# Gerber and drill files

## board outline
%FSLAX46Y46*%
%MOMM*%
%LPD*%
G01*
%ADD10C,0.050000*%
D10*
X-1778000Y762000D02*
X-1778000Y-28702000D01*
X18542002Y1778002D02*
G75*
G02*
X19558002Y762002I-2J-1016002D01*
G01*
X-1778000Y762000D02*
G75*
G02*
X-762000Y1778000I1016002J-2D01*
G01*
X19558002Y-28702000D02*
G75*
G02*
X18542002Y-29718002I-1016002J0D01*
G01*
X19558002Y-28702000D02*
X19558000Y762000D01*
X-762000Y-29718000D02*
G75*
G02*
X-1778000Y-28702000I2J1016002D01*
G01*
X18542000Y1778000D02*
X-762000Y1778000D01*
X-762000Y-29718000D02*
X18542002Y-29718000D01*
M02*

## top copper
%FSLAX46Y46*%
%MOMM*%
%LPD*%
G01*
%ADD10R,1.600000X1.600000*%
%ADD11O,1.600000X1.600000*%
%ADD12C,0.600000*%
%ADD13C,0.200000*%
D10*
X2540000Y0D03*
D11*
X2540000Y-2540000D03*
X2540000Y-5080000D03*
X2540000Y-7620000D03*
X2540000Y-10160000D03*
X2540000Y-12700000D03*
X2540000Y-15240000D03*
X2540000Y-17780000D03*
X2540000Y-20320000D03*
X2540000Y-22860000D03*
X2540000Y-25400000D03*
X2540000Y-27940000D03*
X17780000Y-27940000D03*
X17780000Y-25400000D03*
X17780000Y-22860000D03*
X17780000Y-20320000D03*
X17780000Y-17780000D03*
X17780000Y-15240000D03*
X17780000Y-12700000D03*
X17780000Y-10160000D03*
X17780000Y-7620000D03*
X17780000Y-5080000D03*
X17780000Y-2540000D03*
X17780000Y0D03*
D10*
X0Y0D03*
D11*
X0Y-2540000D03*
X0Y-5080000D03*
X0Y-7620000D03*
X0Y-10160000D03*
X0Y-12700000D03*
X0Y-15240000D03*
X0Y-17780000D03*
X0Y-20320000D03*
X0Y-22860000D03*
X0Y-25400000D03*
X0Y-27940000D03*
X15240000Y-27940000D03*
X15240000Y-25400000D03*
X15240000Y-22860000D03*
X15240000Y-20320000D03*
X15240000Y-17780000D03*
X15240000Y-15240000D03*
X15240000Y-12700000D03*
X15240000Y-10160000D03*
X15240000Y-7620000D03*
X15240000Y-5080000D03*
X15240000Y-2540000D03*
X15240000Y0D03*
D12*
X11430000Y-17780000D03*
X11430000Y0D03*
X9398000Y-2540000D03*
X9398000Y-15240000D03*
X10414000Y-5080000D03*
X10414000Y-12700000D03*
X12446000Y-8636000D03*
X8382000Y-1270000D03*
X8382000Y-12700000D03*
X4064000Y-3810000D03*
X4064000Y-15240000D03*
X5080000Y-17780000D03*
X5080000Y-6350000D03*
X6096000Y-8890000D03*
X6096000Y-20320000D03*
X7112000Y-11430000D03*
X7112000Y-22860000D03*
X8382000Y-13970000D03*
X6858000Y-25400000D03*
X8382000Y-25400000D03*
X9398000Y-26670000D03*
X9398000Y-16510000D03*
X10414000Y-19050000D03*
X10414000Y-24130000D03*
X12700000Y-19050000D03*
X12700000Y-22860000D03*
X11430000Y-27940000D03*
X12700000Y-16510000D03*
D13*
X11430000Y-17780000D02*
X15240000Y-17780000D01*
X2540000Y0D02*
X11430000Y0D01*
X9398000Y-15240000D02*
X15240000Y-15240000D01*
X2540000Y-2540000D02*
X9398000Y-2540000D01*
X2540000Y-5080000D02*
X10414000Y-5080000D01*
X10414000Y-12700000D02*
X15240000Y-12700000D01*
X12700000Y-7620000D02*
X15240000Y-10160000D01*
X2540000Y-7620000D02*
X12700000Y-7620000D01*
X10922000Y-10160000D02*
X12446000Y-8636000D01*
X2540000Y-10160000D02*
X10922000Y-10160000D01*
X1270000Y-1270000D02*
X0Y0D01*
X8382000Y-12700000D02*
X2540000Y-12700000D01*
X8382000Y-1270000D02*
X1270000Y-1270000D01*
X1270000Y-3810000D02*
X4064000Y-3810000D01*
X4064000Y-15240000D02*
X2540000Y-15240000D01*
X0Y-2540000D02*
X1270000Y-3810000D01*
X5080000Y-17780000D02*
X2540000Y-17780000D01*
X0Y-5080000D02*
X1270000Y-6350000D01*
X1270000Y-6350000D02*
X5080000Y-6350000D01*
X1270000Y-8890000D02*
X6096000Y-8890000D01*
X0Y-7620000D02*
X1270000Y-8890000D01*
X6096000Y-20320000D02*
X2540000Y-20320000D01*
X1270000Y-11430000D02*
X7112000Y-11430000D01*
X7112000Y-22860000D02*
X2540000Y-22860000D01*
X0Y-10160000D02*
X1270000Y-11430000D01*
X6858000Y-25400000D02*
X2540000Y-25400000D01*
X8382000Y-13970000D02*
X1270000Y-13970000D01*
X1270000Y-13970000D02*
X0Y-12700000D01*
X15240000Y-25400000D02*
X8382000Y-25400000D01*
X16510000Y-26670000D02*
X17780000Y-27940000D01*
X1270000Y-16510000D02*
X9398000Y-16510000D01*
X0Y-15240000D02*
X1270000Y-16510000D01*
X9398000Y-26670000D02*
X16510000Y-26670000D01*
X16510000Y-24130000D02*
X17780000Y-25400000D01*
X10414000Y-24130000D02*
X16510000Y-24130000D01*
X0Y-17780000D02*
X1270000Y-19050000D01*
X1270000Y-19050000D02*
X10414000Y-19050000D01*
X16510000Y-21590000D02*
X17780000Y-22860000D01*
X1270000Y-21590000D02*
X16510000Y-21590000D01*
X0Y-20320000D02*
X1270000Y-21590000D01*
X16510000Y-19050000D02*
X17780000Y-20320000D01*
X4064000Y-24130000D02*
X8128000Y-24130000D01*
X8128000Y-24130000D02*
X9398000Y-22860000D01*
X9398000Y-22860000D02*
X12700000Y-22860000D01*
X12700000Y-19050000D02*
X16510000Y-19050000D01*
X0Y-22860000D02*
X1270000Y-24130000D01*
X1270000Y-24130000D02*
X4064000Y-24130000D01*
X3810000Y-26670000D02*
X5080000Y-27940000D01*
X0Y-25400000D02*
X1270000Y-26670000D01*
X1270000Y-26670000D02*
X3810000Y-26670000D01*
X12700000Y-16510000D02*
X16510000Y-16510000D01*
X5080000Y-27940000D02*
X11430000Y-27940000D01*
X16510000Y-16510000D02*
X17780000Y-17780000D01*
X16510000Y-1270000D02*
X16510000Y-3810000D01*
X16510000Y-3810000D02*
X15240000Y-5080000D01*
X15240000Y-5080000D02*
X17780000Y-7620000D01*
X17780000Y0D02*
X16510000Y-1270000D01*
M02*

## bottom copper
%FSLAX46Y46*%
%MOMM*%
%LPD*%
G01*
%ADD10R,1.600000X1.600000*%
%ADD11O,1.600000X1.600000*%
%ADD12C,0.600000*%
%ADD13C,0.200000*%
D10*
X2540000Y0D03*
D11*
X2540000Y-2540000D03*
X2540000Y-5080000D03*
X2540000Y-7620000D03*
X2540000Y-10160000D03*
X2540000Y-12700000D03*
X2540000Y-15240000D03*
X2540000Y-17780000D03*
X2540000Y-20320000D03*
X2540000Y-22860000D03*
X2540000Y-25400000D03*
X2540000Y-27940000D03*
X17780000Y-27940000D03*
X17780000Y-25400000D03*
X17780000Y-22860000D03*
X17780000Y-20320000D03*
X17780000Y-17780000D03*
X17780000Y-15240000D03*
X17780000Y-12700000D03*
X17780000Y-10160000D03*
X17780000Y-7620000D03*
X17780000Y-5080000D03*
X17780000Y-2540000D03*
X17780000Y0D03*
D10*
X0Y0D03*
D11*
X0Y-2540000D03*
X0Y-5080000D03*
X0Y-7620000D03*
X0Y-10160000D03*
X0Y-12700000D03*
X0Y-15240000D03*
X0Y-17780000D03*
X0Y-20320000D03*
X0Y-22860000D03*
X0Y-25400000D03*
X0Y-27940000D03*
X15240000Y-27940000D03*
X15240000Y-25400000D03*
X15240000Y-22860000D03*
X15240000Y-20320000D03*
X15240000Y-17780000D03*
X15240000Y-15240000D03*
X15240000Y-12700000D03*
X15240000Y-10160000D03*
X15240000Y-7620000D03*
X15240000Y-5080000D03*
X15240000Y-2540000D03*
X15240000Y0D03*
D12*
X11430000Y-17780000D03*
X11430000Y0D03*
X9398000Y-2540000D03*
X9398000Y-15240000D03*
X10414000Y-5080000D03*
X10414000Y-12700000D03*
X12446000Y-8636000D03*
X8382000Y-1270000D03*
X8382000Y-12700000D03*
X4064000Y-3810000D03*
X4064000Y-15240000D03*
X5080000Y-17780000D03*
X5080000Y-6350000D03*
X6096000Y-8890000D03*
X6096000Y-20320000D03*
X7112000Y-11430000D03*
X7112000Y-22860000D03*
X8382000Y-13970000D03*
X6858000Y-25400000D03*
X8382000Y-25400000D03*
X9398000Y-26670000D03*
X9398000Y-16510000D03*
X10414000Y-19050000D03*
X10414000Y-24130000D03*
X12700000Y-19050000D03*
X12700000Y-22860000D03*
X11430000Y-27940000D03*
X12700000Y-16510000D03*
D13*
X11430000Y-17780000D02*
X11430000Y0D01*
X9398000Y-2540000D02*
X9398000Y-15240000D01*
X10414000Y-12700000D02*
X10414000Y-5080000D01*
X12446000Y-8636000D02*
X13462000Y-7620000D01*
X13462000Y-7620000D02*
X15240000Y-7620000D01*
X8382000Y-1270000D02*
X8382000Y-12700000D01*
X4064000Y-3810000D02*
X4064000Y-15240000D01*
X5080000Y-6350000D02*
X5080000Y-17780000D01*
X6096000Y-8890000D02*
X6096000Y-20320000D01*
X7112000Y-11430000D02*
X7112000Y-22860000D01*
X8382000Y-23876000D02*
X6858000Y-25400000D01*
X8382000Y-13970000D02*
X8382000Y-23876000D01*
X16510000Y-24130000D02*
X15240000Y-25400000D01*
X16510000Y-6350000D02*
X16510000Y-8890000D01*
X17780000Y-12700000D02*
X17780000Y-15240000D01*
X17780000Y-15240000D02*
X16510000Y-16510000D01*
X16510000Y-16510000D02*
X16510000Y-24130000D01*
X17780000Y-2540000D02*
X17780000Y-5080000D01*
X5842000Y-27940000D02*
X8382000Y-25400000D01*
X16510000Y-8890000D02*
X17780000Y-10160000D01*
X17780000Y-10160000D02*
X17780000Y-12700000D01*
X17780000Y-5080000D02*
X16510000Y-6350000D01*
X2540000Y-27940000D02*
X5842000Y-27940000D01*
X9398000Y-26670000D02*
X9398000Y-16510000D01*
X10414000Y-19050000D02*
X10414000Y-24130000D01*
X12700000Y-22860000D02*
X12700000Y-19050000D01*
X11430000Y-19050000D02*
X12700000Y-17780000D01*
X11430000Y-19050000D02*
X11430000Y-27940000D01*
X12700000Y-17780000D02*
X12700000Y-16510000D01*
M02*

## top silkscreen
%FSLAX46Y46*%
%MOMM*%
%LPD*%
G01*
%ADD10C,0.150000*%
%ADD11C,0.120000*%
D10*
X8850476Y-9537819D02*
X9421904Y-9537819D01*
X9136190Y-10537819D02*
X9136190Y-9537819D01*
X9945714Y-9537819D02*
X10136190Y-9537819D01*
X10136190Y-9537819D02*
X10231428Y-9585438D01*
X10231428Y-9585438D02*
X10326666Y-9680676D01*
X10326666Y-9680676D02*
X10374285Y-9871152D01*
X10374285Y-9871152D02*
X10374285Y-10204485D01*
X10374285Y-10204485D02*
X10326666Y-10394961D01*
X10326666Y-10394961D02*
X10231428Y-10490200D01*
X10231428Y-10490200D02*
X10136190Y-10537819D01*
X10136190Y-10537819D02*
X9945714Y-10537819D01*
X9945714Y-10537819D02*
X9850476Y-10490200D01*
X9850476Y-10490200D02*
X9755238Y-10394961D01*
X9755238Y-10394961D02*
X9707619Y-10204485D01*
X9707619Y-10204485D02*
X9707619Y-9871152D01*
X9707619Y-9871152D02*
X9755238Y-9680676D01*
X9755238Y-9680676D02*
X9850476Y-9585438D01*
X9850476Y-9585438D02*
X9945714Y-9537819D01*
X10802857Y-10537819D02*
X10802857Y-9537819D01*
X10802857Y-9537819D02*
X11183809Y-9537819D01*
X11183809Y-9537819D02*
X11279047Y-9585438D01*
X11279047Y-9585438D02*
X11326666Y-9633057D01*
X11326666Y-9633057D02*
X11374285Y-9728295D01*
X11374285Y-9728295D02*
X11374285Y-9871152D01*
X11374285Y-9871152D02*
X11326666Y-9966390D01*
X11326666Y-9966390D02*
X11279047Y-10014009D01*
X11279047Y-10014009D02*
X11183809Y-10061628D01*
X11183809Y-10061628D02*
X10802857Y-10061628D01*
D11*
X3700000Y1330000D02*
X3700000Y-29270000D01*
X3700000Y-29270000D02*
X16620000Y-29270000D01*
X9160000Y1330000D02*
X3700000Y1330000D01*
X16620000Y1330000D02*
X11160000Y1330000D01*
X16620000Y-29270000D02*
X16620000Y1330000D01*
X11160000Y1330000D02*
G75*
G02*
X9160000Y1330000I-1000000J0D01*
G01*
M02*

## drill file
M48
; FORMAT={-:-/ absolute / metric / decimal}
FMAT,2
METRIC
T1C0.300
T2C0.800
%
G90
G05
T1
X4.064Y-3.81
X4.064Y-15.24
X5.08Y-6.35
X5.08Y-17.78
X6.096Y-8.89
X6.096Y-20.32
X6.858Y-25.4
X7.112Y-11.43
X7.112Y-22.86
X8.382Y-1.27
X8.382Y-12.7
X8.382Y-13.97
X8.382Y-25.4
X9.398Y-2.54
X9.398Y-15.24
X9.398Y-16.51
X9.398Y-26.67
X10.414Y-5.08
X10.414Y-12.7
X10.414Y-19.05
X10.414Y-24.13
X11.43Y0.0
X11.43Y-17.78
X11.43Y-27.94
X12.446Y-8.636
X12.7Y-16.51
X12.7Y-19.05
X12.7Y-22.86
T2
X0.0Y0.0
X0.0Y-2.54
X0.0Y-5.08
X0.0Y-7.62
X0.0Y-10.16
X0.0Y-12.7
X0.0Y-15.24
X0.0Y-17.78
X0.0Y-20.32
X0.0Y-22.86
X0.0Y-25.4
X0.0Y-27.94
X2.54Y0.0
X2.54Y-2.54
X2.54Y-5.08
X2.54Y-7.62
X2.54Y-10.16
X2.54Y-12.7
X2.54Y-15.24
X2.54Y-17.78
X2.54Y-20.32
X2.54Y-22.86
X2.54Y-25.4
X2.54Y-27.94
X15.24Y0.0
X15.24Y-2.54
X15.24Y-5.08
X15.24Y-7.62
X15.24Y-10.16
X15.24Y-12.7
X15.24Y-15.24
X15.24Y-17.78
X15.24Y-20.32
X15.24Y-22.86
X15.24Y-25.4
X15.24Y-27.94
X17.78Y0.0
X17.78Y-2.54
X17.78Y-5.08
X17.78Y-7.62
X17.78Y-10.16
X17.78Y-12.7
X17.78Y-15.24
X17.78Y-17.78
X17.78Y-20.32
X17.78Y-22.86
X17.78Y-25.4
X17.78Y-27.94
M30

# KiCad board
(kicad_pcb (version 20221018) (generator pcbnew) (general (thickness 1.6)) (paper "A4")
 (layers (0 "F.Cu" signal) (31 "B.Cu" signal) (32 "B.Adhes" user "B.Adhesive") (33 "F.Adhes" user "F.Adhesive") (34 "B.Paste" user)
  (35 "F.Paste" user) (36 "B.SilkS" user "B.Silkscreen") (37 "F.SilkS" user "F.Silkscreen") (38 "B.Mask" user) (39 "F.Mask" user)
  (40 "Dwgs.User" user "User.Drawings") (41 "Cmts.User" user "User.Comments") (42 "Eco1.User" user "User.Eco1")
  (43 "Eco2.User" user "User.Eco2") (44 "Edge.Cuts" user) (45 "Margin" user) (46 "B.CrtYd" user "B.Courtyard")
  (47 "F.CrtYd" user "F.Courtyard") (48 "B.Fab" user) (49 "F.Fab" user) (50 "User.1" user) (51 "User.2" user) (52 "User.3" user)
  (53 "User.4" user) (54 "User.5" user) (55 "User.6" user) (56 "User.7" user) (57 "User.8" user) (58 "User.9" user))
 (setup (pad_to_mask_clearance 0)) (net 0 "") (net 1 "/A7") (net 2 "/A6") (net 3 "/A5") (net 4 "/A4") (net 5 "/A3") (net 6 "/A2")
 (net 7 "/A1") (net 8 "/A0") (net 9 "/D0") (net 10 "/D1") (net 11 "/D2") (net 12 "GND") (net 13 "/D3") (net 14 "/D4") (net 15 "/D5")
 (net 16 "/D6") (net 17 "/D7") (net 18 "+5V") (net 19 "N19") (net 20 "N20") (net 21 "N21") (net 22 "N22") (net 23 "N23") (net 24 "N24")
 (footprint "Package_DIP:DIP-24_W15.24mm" (layer "F.Cu") (at 2.54 0)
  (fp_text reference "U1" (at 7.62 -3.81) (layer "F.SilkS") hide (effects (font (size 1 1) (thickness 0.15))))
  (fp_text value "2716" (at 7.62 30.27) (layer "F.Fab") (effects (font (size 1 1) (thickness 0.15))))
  (fp_line (start 1.16 -1.33) (end 1.16 29.27) (stroke (width 0.12) (type solid)) (layer "F.SilkS"))
  (fp_line (start 1.16 29.27) (end 14.08 29.27) (stroke (width 0.12) (type solid)) (layer "F.SilkS"))
  (fp_line (start 6.62 -1.33) (end 1.16 -1.33) (stroke (width 0.12) (type solid)) (layer "F.SilkS"))
  (fp_line (start 14.08 -1.33) (end 8.62 -1.33) (stroke (width 0.12) (type solid)) (layer "F.SilkS"))
  (fp_line (start 14.08 29.27) (end 14.08 -1.33) (stroke (width 0.12) (type solid)) (layer "F.SilkS"))
  (fp_arc (start 8.62 -1.33) (mid 7.62 -0.33) (end 6.62 -1.33) (stroke (width 0.12) (type solid)) (layer "F.SilkS"))
  (pad "1" thru_hole rect (at 0 0) (size 1.6 1.6) (drill 0.8) (layers "*.Cu" "*.Mask") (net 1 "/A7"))
  (pad "2" thru_hole oval (at 0 2.54) (size 1.6 1.6) (drill 0.8) (layers "*.Cu" "*.Mask") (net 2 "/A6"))
  (pad "3" thru_hole oval (at 0 5.08) (size 1.6 1.6) (drill 0.8) (layers "*.Cu" "*.Mask") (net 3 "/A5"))
  (pad "4" thru_hole oval (at 0 7.62) (size 1.6 1.6) (drill 0.8) (layers "*.Cu" "*.Mask") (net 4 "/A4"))
  (pad "5" thru_hole oval (at 0 10.16) (size 1.6 1.6) (drill 0.8) (layers "*.Cu" "*.Mask") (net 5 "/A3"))
  (pad "6" thru_hole oval (at 0 12.7) (size 1.6 1.6) (drill 0.8) (layers "*.Cu" "*.Mask") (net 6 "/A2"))
  (pad "7" thru_hole oval (at 0 15.24) (size 1.6 1.6) (drill 0.8) (layers "*.Cu" "*.Mask") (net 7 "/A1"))
  (pad "8" thru_hole oval (at 0 17.78) (size 1.6 1.6) (drill 0.8) (layers "*.Cu" "*.Mask") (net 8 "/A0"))
  (pad "9" thru_hole oval (at 0 20.32) (size 1.6 1.6) (drill 0.8) (layers "*.Cu" "*.Mask") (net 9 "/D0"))
  (pad "10" thru_hole oval (at 0 22.86) (size 1.6 1.6) (drill 0.8) (layers "*.Cu" "*.Mask") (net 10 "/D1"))
  (pad "11" thru_hole oval (at 0 25.4) (size 1.6 1.6) (drill 0.8) (layers "*.Cu" "*.Mask") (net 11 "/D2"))
  (pad "12" thru_hole oval (at 0 27.94) (size 1.6 1.6) (drill 0.8) (layers "*.Cu" "*.Mask") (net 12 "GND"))
  (pad "13" thru_hole oval (at 15.24 27.94) (size 1.6 1.6) (drill 0.8) (layers "*.Cu" "*.Mask") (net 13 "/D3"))
  (pad "14" thru_hole oval (at 15.24 25.4) (size 1.6 1.6) (drill 0.8) (layers "*.Cu" "*.Mask") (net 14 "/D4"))
  (pad "15" thru_hole oval (at 15.24 22.86) (size 1.6 1.6) (drill 0.8) (layers "*.Cu" "*.Mask") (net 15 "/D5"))
  (pad "16" thru_hole oval (at 15.24 20.32) (size 1.6 1.6) (drill 0.8) (layers "*.Cu" "*.Mask") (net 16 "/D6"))
  (pad "17" thru_hole oval (at 15.24 17.78) (size 1.6 1.6) (drill 0.8) (layers "*.Cu" "*.Mask") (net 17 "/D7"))
  (pad "18" thru_hole oval (at 15.24 15.24) (size 1.6 1.6) (drill 0.8) (layers "*.Cu" "*.Mask") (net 12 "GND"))
  (pad "19" thru_hole oval (at 15.24 12.7) (size 1.6 1.6) (drill 0.8) (layers "*.Cu" "*.Mask") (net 12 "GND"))
  (pad "20" thru_hole oval (at 15.24 10.16) (size 1.6 1.6) (drill 0.8) (layers "*.Cu" "*.Mask") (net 12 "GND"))
  (pad "21" thru_hole oval (at 15.24 7.62) (size 1.6 1.6) (drill 0.8) (layers "*.Cu" "*.Mask") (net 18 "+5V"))
  (pad "22" thru_hole oval (at 15.24 5.08) (size 1.6 1.6) (drill 0.8) (layers "*.Cu" "*.Mask") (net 12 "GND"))
  (pad "23" thru_hole oval (at 15.24 2.54) (size 1.6 1.6) (drill 0.8) (layers "*.Cu" "*.Mask") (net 12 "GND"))
  (pad "24" thru_hole oval (at 15.24 0) (size 1.6 1.6) (drill 0.8) (layers "*.Cu" "*.Mask") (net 18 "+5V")))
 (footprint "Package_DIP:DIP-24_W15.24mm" (layer "F.Cu") (at 0 0)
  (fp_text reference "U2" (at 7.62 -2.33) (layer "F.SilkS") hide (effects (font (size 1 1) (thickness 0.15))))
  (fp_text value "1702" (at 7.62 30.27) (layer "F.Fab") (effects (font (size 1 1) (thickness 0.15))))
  (pad "1" thru_hole rect (at 0 0) (size 1.6 1.6) (drill 0.8) (layers "*.Cu" "*.Mask") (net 6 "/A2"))
  (pad "2" thru_hole oval (at 0 2.54) (size 1.6 1.6) (drill 0.8) (layers "*.Cu" "*.Mask") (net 7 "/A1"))
  (pad "3" thru_hole oval (at 0 5.08) (size 1.6 1.6) (drill 0.8) (layers "*.Cu" "*.Mask") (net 8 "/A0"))
  (pad "4" thru_hole oval (at 0 7.62) (size 1.6 1.6) (drill 0.8) (layers "*.Cu" "*.Mask") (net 9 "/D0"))
  (pad "5" thru_hole oval (at 0 10.16) (size 1.6 1.6) (drill 0.8) (layers "*.Cu" "*.Mask") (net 10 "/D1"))
  (pad "6" thru_hole oval (at 0 12.7) (size 1.6 1.6) (drill 0.8) (layers "*.Cu" "*.Mask") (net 11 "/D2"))
  (pad "7" thru_hole oval (at 0 15.24) (size 1.6 1.6) (drill 0.8) (layers "*.Cu" "*.Mask") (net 13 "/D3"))
  (pad "8" thru_hole oval (at 0 17.78) (size 1.6 1.6) (drill 0.8) (layers "*.Cu" "*.Mask") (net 14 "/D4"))
  (pad "9" thru_hole oval (at 0 20.32) (size 1.6 1.6) (drill 0.8) (layers "*.Cu" "*.Mask") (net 15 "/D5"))
  (pad "10" thru_hole oval (at 0 22.86) (size 1.6 1.6) (drill 0.8) (layers "*.Cu" "*.Mask") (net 16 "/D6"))
  (pad "11" thru_hole oval (at 0 25.4) (size 1.6 1.6) (drill 0.8) (layers "*.Cu" "*.Mask") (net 17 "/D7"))
  (pad "12" thru_hole oval (at 0 27.94) (size 1.6 1.6) (drill 0.8) (layers "*.Cu" "*.Mask") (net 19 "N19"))
  (pad "13" thru_hole oval (at 15.24 27.94) (size 1.6 1.6) (drill 0.8) (layers "*.Cu" "*.Mask") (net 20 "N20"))
  (pad "14" thru_hole oval (at 15.24 25.4) (size 1.6 1.6) (drill 0.8) (layers "*.Cu" "*.Mask") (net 12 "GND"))
  (pad "15" thru_hole oval (at 15.24 22.86) (size 1.6 1.6) (drill 0.8) (layers "*.Cu" "*.Mask") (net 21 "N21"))
  (pad "16" thru_hole oval (at 15.24 20.32) (size 1.6 1.6) (drill 0.8) (layers "*.Cu" "*.Mask") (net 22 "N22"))
  (pad "17" thru_hole oval (at 15.24 17.78) (size 1.6 1.6) (drill 0.8) (layers "*.Cu" "*.Mask") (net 1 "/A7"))
  (pad "18" thru_hole oval (at 15.24 15.24) (size 1.6 1.6) (drill 0.8) (layers "*.Cu" "*.Mask") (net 2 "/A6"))
  (pad "19" thru_hole oval (at 15.24 12.7) (size 1.6 1.6) (drill 0.8) (layers "*.Cu" "*.Mask") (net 3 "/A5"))
  (pad "20" thru_hole oval (at 15.24 10.16) (size 1.6 1.6) (drill 0.8) (layers "*.Cu" "*.Mask") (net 4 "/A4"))
  (pad "21" thru_hole oval (at 15.24 7.62) (size 1.6 1.6) (drill 0.8) (layers "*.Cu" "*.Mask") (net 5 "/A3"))
  (pad "22" thru_hole oval (at 15.24 5.08) (size 1.6 1.6) (drill 0.8) (layers "*.Cu" "*.Mask") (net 18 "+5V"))
  (pad "23" thru_hole oval (at 15.24 2.54) (size 1.6 1.6) (drill 0.8) (layers "*.Cu" "*.Mask") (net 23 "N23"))
  (pad "24" thru_hole oval (at 15.24 0) (size 1.6 1.6) (drill 0.8) (layers "*.Cu" "*.Mask") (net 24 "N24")))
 (gr_line (start -1.778 -0.762) (end -1.778 28.702) (stroke (width 0.05) (type default)) (layer "Edge.Cuts"))
 (gr_arc (start 18.542002 -1.778002) (mid 19.260422 -1.480422) (end 19.558002 -0.762002) (stroke (width 0.05) (type default))
  (layer "Edge.Cuts"))
 (gr_arc (start -1.778 -0.762) (mid -1.48042 -1.48042) (end -0.762 -1.778) (stroke (width 0.05) (type default)) (layer "Edge.Cuts"))
 (gr_arc (start 19.558002 28.702) (mid 19.260422 29.42042) (end 18.542002 29.718) (stroke (width 0.05) (type default)) (layer "Edge.Cuts"))
 (gr_line (start 19.558002 28.702) (end 19.558 -0.762) (stroke (width 0.05) (type default)) (layer "Edge.Cuts"))
 (gr_arc (start -0.762 29.718) (mid -1.48042 29.42042) (end -1.778 28.702) (stroke (width 0.05) (type default)) (layer "Edge.Cuts"))
 (gr_line (start 18.542 -1.778) (end -0.762 -1.778) (stroke (width 0.05) (type default)) (layer "Edge.Cuts"))
 (gr_line (start -0.762 29.718) (end 18.542002 29.718) (stroke (width 0.05) (type default)) (layer "Edge.Cuts"))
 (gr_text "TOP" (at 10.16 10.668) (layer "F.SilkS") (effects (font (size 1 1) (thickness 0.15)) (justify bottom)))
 (segment (start 11.43 17.78) (end 15.24 17.78) (width 0.2) (layer "F.Cu") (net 1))
 (segment (start 2.54 0) (end 11.43 0) (width 0.2) (layer "F.Cu") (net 1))
 (via (at 11.43 17.78) (size 0.6) (drill 0.3) (layers "F.Cu" "B.Cu") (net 1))
 (via (at 11.43 0) (size 0.6) (drill 0.3) (layers "F.Cu" "B.Cu") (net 1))
 (segment (start 11.43 17.78) (end 11.43 0) (width 0.2) (layer "B.Cu") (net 1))
 (segment (start 9.398 15.24) (end 15.24 15.24) (width 0.2) (layer "F.Cu") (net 2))
 (segment (start 2.54 2.54) (end 9.398 2.54) (width 0.2) (layer "F.Cu") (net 2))
 (via (at 9.398 2.54) (size 0.6) (drill 0.3) (layers "F.Cu" "B.Cu") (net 2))
 (via (at 9.398 15.24) (size 0.6) (drill 0.3) (layers "F.Cu" "B.Cu") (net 2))
 (segment (start 9.398 2.54) (end 9.398 15.24) (width 0.2) (layer "B.Cu") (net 2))
 (segment (start 2.54 5.08) (end 10.414 5.08) (width 0.2) (layer "F.Cu") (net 3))
 (segment (start 10.414 12.7) (end 15.24 12.7) (width 0.2) (layer "F.Cu") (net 3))
 (via (at 10.414 5.08) (size 0.6) (drill 0.3) (layers "F.Cu" "B.Cu") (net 3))
 (via (at 10.414 12.7) (size 0.6) (drill 0.3) (layers "F.Cu" "B.Cu") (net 3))
 (segment (start 10.414 12.7) (end 10.414 5.08) (width 0.2) (layer "B.Cu") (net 3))
 (segment (start 12.7 7.62) (end 15.24 10.16) (width 0.2) (layer "F.Cu") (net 4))
 (segment (start 2.54 7.62) (end 12.7 7.62) (width 0.2) (layer "F.Cu") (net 4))
 (segment (start 10.922 10.16) (end 12.446 8.636) (width 0.2) (layer "F.Cu") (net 5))
 (segment (start 2.54 10.16) (end 10.922 10.16) (width 0.2) (layer "F.Cu") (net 5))
 (via (at 12.446 8.636) (size 0.6) (drill 0.3) (layers "F.Cu" "B.Cu") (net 5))
 (segment (start 12.446 8.636) (end 13.462 7.62) (width 0.2) (layer "B.Cu") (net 5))
 (segment (start 13.462 7.62) (end 15.24 7.62) (width 0.2) (layer "B.Cu") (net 5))
 (segment (start 1.27 1.27) (end 0 0) (width 0.2) (layer "F.Cu") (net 6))
 (segment (start 8.382 12.7) (end 2.54 12.7) (width 0.2) (layer "F.Cu") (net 6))
 (segment (start 8.382 1.27) (end 1.27 1.27) (width 0.2) (layer "F.Cu") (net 6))
 (via (at 8.382 1.27) (size 0.6) (drill 0.3) (layers "F.Cu" "B.Cu") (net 6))
 (via (at 8.382 12.7) (size 0.6) (drill 0.3) (layers "F.Cu" "B.Cu") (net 6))
 (segment (start 8.382 1.27) (end 8.382 12.7) (width 0.2) (layer "B.Cu") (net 6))
 (segment (start 1.27 3.81) (end 4.064 3.81) (width 0.2) (layer "F.Cu") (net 7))
 (segment (start 4.064 15.24) (end 2.54 15.24) (width 0.2) (layer "F.Cu") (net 7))
 (segment (start 0 2.54) (end 1.27 3.81) (width 0.2) (layer "F.Cu") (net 7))
 (via (at 4.064 3.81) (size 0.6) (drill 0.3) (layers "F.Cu" "B.Cu") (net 7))
 (via (at 4.064 15.24) (size 0.6) (drill 0.3) (layers "F.Cu" "B.Cu") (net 7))
 (segment (start 4.064 3.81) (end 4.064 15.24) (width 0.2) (layer "B.Cu") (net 7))
 (segment (start 5.08 17.78) (end 2.54 17.78) (width 0.2) (layer "F.Cu") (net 8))
 (segment (start 0 5.08) (end 1.27 6.35) (width 0.2) (layer "F.Cu") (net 8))
 (segment (start 1.27 6.35) (end 5.08 6.35) (width 0.2) (layer "F.Cu") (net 8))
 (via (at 5.08 17.78) (size 0.6) (drill 0.3) (layers "F.Cu" "B.Cu") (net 8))
 (via (at 5.08 6.35) (size 0.6) (drill 0.3) (layers "F.Cu" "B.Cu") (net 8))
 (segment (start 5.08 6.35) (end 5.08 17.78) (width 0.2) (layer "B.Cu") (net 8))
 (segment (start 1.27 8.89) (end 6.096 8.89) (width 0.2) (layer "F.Cu") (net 9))
 (segment (start 0 7.62) (end 1.27 8.89) (width 0.2) (layer "F.Cu") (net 9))
 (segment (start 6.096 20.32) (end 2.54 20.32) (width 0.2) (layer "F.Cu") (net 9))
 (via (at 6.096 8.89) (size 0.6) (drill 0.3) (layers "F.Cu" "B.Cu") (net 9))
 (via (at 6.096 20.32) (size 0.6) (drill 0.3) (layers "F.Cu" "B.Cu") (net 9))
 (segment (start 6.096 8.89) (end 6.096 20.32) (width 0.2) (layer "B.Cu") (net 9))
 (segment (start 1.27 11.43) (end 7.112 11.43) (width 0.2) (layer "F.Cu") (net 10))
 (segment (start 7.112 22.86) (end 2.54 22.86) (width 0.2) (layer "F.Cu") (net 10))
 (segment (start 0 10.16) (end 1.27 11.43) (width 0.2) (layer "F.Cu") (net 10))
 (via (at 7.112 11.43) (size 0.6) (drill 0.3) (layers "F.Cu" "B.Cu") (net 10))
 (via (at 7.112 22.86) (size 0.6) (drill 0.3) (layers "F.Cu" "B.Cu") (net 10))
 (segment (start 7.112 11.43) (end 7.112 22.86) (width 0.2) (layer "B.Cu") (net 10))
 (segment (start 6.858 25.4) (end 2.54 25.4) (width 0.2) (layer "F.Cu") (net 11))
 (segment (start 8.382 13.97) (end 1.27 13.97) (width 0.2) (layer "F.Cu") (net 11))
 (segment (start 1.27 13.97) (end 0 12.7) (width 0.2) (layer "F.Cu") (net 11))
 (via (at 8.382 13.97) (size 0.6) (drill 0.3) (layers "F.Cu" "B.Cu") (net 11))
 (via (at 6.858 25.4) (size 0.6) (drill 0.3) (layers "F.Cu" "B.Cu") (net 11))
 (segment (start 8.382 23.876) (end 6.858 25.4) (width 0.2) (layer "B.Cu") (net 11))
 (segment (start 8.382 13.97) (end 8.382 23.876) (width 0.2) (layer "B.Cu") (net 11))
 (segment (start 15.24 25.4) (end 8.382 25.4) (width 0.2) (layer "F.Cu") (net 12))
 (via (at 8.382 25.4) (size 0.6) (drill 0.3) (layers "F.Cu" "B.Cu") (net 12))
 (segment (start 16.51 24.13) (end 15.24 25.4) (width 0.2) (layer "B.Cu") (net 12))
 (segment (start 16.51 6.35) (end 16.51 8.89) (width 0.2) (layer "B.Cu") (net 12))
 (segment (start 17.78 12.7) (end 17.78 15.24) (width 0.2) (layer "B.Cu") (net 12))
 (segment (start 17.78 15.24) (end 16.51 16.51) (width 0.2) (layer "B.Cu") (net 12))
 (segment (start 16.51 16.51) (end 16.51 24.13) (width 0.2) (layer "B.Cu") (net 12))
 (segment (start 17.78 2.54) (end 17.78 5.08) (width 0.2) (layer "B.Cu") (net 12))
 (segment (start 5.842 27.94) (end 8.382 25.4) (width 0.2) (layer "B.Cu") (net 12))
 (segment (start 16.51 8.89) (end 17.78 10.16) (width 0.2) (layer "B.Cu") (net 12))
 (segment (start 17.78 10.16) (end 17.78 12.7) (width 0.2) (layer "B.Cu") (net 12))
 (segment (start 17.78 5.08) (end 16.51 6.35) (width 0.2) (layer "B.Cu") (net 12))
 (segment (start 2.54 27.94) (end 5.842 27.94) (width 0.2) (layer "B.Cu") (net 12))
 (segment (start 16.51 26.67) (end 17.78 27.94) (width 0.2) (layer "F.Cu") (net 13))
 (segment (start 1.27 16.51) (end 9.398 16.51) (width 0.2) (layer "F.Cu") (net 13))
 (segment (start 0 15.24) (end 1.27 16.51) (width 0.2) (layer "F.Cu") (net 13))
 (segment (start 9.398 26.67) (end 16.51 26.67) (width 0.2) (layer "F.Cu") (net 13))
 (via (at 9.398 26.67) (size 0.6) (drill 0.3) (layers "F.Cu" "B.Cu") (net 13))
 (via (at 9.398 16.51) (size 0.6) (drill 0.3) (layers "F.Cu" "B.Cu") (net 13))
 (segment (start 9.398 26.67) (end 9.398 16.51) (width 0.2) (layer "B.Cu") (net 13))
 (segment (start 16.51 24.13) (end 17.78 25.4) (width 0.2) (layer "F.Cu") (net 14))
 (segment (start 10.414 24.13) (end 16.51 24.13) (width 0.2) (layer "F.Cu") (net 14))
 (segment (start 0 17.78) (end 1.27 19.05) (width 0.2) (layer "F.Cu") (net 14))
 (segment (start 1.27 19.05) (end 10.414 19.05) (width 0.2) (layer "F.Cu") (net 14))
 (via (at 10.414 19.05) (size 0.6) (drill 0.3) (layers "F.Cu" "B.Cu") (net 14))
 (via (at 10.414 24.13) (size 0.6) (drill 0.3) (layers "F.Cu" "B.Cu") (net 14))
 (segment (start 10.414 19.05) (end 10.414 24.13) (width 0.2) (layer "B.Cu") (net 14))
 (segment (start 16.51 21.59) (end 17.78 22.86) (width 0.2) (layer "F.Cu") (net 15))
 (segment (start 1.27 21.59) (end 16.51 21.59) (width 0.2) (layer "F.Cu") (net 15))
 (segment (start 0 20.32) (end 1.27 21.59) (width 0.2) (layer "F.Cu") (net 15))
 (segment (start 16.51 19.05) (end 17.78 20.32) (width 0.2) (layer "F.Cu") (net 16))
 (segment (start 4.064 24.13) (end 8.128 24.13) (width 0.2) (layer "F.Cu") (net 16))
 (segment (start 8.128 24.13) (end 9.398 22.86) (width 0.2) (layer "F.Cu") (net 16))
 (segment (start 9.398 22.86) (end 12.7 22.86) (width 0.2) (layer "F.Cu") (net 16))
 (segment (start 12.7 19.05) (end 16.51 19.05) (width 0.2) (layer "F.Cu") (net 16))
 (segment (start 0 22.86) (end 1.27 24.13) (width 0.2) (layer "F.Cu") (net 16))
 (segment (start 1.27 24.13) (end 4.064 24.13) (width 0.2) (layer "F.Cu") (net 16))
 (via (at 12.7 19.05) (size 0.6) (drill 0.3) (layers "F.Cu" "B.Cu") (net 16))
 (via (at 12.7 22.86) (size 0.6) (drill 0.3) (layers "F.Cu" "B.Cu") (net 16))
 (segment (start 12.7 22.86) (end 12.7 19.05) (width 0.2) (layer "B.Cu") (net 16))
 (segment (start 3.81 26.67) (end 5.08 27.94) (width 0.2) (layer "F.Cu") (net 17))
 (segment (start 0 25.4) (end 1.27 26.67) (width 0.2) (layer "F.Cu") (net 17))
 (segment (start 1.27 26.67) (end 3.81 26.67) (width 0.2) (layer "F.Cu") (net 17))
 (segment (start 12.7 16.51) (end 16.51 16.51) (width 0.2) (layer "F.Cu") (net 17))
 (segment (start 5.08 27.94) (end 11.43 27.94) (width 0.2) (layer "F.Cu") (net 17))
 (segment (start 16.51 16.51) (end 17.78 17.78) (width 0.2) (layer "F.Cu") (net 17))
 (via (at 11.43 27.94) (size 0.6) (drill 0.3) (layers "F.Cu" "B.Cu") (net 17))
 (via (at 12.7 16.51) (size 0.6) (drill 0.3) (layers "F.Cu" "B.Cu") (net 17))
 (segment (start 11.43 19.05) (end 12.7 17.78) (width 0.2) (layer "B.Cu") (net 17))
 (segment (start 11.43 19.05) (end 11.43 27.94) (width 0.2) (layer "B.Cu") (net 17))
 (segment (start 12.7 17.78) (end 12.7 16.51) (width 0.2) (layer "B.Cu") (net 17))
 (segment (start 16.51 1.27) (end 16.51 3.81) (width 0.2) (layer "F.Cu") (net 18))
 (segment (start 16.51 3.81) (end 15.24 5.08) (width 0.2) (layer "F.Cu") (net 18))
 (segment (start 15.24 5.08) (end 17.78 7.62) (width 0.2) (layer "F.Cu") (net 18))
 (segment (start 17.78 0) (end 16.51 1.27) (width 0.2) (layer "F.Cu") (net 18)))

